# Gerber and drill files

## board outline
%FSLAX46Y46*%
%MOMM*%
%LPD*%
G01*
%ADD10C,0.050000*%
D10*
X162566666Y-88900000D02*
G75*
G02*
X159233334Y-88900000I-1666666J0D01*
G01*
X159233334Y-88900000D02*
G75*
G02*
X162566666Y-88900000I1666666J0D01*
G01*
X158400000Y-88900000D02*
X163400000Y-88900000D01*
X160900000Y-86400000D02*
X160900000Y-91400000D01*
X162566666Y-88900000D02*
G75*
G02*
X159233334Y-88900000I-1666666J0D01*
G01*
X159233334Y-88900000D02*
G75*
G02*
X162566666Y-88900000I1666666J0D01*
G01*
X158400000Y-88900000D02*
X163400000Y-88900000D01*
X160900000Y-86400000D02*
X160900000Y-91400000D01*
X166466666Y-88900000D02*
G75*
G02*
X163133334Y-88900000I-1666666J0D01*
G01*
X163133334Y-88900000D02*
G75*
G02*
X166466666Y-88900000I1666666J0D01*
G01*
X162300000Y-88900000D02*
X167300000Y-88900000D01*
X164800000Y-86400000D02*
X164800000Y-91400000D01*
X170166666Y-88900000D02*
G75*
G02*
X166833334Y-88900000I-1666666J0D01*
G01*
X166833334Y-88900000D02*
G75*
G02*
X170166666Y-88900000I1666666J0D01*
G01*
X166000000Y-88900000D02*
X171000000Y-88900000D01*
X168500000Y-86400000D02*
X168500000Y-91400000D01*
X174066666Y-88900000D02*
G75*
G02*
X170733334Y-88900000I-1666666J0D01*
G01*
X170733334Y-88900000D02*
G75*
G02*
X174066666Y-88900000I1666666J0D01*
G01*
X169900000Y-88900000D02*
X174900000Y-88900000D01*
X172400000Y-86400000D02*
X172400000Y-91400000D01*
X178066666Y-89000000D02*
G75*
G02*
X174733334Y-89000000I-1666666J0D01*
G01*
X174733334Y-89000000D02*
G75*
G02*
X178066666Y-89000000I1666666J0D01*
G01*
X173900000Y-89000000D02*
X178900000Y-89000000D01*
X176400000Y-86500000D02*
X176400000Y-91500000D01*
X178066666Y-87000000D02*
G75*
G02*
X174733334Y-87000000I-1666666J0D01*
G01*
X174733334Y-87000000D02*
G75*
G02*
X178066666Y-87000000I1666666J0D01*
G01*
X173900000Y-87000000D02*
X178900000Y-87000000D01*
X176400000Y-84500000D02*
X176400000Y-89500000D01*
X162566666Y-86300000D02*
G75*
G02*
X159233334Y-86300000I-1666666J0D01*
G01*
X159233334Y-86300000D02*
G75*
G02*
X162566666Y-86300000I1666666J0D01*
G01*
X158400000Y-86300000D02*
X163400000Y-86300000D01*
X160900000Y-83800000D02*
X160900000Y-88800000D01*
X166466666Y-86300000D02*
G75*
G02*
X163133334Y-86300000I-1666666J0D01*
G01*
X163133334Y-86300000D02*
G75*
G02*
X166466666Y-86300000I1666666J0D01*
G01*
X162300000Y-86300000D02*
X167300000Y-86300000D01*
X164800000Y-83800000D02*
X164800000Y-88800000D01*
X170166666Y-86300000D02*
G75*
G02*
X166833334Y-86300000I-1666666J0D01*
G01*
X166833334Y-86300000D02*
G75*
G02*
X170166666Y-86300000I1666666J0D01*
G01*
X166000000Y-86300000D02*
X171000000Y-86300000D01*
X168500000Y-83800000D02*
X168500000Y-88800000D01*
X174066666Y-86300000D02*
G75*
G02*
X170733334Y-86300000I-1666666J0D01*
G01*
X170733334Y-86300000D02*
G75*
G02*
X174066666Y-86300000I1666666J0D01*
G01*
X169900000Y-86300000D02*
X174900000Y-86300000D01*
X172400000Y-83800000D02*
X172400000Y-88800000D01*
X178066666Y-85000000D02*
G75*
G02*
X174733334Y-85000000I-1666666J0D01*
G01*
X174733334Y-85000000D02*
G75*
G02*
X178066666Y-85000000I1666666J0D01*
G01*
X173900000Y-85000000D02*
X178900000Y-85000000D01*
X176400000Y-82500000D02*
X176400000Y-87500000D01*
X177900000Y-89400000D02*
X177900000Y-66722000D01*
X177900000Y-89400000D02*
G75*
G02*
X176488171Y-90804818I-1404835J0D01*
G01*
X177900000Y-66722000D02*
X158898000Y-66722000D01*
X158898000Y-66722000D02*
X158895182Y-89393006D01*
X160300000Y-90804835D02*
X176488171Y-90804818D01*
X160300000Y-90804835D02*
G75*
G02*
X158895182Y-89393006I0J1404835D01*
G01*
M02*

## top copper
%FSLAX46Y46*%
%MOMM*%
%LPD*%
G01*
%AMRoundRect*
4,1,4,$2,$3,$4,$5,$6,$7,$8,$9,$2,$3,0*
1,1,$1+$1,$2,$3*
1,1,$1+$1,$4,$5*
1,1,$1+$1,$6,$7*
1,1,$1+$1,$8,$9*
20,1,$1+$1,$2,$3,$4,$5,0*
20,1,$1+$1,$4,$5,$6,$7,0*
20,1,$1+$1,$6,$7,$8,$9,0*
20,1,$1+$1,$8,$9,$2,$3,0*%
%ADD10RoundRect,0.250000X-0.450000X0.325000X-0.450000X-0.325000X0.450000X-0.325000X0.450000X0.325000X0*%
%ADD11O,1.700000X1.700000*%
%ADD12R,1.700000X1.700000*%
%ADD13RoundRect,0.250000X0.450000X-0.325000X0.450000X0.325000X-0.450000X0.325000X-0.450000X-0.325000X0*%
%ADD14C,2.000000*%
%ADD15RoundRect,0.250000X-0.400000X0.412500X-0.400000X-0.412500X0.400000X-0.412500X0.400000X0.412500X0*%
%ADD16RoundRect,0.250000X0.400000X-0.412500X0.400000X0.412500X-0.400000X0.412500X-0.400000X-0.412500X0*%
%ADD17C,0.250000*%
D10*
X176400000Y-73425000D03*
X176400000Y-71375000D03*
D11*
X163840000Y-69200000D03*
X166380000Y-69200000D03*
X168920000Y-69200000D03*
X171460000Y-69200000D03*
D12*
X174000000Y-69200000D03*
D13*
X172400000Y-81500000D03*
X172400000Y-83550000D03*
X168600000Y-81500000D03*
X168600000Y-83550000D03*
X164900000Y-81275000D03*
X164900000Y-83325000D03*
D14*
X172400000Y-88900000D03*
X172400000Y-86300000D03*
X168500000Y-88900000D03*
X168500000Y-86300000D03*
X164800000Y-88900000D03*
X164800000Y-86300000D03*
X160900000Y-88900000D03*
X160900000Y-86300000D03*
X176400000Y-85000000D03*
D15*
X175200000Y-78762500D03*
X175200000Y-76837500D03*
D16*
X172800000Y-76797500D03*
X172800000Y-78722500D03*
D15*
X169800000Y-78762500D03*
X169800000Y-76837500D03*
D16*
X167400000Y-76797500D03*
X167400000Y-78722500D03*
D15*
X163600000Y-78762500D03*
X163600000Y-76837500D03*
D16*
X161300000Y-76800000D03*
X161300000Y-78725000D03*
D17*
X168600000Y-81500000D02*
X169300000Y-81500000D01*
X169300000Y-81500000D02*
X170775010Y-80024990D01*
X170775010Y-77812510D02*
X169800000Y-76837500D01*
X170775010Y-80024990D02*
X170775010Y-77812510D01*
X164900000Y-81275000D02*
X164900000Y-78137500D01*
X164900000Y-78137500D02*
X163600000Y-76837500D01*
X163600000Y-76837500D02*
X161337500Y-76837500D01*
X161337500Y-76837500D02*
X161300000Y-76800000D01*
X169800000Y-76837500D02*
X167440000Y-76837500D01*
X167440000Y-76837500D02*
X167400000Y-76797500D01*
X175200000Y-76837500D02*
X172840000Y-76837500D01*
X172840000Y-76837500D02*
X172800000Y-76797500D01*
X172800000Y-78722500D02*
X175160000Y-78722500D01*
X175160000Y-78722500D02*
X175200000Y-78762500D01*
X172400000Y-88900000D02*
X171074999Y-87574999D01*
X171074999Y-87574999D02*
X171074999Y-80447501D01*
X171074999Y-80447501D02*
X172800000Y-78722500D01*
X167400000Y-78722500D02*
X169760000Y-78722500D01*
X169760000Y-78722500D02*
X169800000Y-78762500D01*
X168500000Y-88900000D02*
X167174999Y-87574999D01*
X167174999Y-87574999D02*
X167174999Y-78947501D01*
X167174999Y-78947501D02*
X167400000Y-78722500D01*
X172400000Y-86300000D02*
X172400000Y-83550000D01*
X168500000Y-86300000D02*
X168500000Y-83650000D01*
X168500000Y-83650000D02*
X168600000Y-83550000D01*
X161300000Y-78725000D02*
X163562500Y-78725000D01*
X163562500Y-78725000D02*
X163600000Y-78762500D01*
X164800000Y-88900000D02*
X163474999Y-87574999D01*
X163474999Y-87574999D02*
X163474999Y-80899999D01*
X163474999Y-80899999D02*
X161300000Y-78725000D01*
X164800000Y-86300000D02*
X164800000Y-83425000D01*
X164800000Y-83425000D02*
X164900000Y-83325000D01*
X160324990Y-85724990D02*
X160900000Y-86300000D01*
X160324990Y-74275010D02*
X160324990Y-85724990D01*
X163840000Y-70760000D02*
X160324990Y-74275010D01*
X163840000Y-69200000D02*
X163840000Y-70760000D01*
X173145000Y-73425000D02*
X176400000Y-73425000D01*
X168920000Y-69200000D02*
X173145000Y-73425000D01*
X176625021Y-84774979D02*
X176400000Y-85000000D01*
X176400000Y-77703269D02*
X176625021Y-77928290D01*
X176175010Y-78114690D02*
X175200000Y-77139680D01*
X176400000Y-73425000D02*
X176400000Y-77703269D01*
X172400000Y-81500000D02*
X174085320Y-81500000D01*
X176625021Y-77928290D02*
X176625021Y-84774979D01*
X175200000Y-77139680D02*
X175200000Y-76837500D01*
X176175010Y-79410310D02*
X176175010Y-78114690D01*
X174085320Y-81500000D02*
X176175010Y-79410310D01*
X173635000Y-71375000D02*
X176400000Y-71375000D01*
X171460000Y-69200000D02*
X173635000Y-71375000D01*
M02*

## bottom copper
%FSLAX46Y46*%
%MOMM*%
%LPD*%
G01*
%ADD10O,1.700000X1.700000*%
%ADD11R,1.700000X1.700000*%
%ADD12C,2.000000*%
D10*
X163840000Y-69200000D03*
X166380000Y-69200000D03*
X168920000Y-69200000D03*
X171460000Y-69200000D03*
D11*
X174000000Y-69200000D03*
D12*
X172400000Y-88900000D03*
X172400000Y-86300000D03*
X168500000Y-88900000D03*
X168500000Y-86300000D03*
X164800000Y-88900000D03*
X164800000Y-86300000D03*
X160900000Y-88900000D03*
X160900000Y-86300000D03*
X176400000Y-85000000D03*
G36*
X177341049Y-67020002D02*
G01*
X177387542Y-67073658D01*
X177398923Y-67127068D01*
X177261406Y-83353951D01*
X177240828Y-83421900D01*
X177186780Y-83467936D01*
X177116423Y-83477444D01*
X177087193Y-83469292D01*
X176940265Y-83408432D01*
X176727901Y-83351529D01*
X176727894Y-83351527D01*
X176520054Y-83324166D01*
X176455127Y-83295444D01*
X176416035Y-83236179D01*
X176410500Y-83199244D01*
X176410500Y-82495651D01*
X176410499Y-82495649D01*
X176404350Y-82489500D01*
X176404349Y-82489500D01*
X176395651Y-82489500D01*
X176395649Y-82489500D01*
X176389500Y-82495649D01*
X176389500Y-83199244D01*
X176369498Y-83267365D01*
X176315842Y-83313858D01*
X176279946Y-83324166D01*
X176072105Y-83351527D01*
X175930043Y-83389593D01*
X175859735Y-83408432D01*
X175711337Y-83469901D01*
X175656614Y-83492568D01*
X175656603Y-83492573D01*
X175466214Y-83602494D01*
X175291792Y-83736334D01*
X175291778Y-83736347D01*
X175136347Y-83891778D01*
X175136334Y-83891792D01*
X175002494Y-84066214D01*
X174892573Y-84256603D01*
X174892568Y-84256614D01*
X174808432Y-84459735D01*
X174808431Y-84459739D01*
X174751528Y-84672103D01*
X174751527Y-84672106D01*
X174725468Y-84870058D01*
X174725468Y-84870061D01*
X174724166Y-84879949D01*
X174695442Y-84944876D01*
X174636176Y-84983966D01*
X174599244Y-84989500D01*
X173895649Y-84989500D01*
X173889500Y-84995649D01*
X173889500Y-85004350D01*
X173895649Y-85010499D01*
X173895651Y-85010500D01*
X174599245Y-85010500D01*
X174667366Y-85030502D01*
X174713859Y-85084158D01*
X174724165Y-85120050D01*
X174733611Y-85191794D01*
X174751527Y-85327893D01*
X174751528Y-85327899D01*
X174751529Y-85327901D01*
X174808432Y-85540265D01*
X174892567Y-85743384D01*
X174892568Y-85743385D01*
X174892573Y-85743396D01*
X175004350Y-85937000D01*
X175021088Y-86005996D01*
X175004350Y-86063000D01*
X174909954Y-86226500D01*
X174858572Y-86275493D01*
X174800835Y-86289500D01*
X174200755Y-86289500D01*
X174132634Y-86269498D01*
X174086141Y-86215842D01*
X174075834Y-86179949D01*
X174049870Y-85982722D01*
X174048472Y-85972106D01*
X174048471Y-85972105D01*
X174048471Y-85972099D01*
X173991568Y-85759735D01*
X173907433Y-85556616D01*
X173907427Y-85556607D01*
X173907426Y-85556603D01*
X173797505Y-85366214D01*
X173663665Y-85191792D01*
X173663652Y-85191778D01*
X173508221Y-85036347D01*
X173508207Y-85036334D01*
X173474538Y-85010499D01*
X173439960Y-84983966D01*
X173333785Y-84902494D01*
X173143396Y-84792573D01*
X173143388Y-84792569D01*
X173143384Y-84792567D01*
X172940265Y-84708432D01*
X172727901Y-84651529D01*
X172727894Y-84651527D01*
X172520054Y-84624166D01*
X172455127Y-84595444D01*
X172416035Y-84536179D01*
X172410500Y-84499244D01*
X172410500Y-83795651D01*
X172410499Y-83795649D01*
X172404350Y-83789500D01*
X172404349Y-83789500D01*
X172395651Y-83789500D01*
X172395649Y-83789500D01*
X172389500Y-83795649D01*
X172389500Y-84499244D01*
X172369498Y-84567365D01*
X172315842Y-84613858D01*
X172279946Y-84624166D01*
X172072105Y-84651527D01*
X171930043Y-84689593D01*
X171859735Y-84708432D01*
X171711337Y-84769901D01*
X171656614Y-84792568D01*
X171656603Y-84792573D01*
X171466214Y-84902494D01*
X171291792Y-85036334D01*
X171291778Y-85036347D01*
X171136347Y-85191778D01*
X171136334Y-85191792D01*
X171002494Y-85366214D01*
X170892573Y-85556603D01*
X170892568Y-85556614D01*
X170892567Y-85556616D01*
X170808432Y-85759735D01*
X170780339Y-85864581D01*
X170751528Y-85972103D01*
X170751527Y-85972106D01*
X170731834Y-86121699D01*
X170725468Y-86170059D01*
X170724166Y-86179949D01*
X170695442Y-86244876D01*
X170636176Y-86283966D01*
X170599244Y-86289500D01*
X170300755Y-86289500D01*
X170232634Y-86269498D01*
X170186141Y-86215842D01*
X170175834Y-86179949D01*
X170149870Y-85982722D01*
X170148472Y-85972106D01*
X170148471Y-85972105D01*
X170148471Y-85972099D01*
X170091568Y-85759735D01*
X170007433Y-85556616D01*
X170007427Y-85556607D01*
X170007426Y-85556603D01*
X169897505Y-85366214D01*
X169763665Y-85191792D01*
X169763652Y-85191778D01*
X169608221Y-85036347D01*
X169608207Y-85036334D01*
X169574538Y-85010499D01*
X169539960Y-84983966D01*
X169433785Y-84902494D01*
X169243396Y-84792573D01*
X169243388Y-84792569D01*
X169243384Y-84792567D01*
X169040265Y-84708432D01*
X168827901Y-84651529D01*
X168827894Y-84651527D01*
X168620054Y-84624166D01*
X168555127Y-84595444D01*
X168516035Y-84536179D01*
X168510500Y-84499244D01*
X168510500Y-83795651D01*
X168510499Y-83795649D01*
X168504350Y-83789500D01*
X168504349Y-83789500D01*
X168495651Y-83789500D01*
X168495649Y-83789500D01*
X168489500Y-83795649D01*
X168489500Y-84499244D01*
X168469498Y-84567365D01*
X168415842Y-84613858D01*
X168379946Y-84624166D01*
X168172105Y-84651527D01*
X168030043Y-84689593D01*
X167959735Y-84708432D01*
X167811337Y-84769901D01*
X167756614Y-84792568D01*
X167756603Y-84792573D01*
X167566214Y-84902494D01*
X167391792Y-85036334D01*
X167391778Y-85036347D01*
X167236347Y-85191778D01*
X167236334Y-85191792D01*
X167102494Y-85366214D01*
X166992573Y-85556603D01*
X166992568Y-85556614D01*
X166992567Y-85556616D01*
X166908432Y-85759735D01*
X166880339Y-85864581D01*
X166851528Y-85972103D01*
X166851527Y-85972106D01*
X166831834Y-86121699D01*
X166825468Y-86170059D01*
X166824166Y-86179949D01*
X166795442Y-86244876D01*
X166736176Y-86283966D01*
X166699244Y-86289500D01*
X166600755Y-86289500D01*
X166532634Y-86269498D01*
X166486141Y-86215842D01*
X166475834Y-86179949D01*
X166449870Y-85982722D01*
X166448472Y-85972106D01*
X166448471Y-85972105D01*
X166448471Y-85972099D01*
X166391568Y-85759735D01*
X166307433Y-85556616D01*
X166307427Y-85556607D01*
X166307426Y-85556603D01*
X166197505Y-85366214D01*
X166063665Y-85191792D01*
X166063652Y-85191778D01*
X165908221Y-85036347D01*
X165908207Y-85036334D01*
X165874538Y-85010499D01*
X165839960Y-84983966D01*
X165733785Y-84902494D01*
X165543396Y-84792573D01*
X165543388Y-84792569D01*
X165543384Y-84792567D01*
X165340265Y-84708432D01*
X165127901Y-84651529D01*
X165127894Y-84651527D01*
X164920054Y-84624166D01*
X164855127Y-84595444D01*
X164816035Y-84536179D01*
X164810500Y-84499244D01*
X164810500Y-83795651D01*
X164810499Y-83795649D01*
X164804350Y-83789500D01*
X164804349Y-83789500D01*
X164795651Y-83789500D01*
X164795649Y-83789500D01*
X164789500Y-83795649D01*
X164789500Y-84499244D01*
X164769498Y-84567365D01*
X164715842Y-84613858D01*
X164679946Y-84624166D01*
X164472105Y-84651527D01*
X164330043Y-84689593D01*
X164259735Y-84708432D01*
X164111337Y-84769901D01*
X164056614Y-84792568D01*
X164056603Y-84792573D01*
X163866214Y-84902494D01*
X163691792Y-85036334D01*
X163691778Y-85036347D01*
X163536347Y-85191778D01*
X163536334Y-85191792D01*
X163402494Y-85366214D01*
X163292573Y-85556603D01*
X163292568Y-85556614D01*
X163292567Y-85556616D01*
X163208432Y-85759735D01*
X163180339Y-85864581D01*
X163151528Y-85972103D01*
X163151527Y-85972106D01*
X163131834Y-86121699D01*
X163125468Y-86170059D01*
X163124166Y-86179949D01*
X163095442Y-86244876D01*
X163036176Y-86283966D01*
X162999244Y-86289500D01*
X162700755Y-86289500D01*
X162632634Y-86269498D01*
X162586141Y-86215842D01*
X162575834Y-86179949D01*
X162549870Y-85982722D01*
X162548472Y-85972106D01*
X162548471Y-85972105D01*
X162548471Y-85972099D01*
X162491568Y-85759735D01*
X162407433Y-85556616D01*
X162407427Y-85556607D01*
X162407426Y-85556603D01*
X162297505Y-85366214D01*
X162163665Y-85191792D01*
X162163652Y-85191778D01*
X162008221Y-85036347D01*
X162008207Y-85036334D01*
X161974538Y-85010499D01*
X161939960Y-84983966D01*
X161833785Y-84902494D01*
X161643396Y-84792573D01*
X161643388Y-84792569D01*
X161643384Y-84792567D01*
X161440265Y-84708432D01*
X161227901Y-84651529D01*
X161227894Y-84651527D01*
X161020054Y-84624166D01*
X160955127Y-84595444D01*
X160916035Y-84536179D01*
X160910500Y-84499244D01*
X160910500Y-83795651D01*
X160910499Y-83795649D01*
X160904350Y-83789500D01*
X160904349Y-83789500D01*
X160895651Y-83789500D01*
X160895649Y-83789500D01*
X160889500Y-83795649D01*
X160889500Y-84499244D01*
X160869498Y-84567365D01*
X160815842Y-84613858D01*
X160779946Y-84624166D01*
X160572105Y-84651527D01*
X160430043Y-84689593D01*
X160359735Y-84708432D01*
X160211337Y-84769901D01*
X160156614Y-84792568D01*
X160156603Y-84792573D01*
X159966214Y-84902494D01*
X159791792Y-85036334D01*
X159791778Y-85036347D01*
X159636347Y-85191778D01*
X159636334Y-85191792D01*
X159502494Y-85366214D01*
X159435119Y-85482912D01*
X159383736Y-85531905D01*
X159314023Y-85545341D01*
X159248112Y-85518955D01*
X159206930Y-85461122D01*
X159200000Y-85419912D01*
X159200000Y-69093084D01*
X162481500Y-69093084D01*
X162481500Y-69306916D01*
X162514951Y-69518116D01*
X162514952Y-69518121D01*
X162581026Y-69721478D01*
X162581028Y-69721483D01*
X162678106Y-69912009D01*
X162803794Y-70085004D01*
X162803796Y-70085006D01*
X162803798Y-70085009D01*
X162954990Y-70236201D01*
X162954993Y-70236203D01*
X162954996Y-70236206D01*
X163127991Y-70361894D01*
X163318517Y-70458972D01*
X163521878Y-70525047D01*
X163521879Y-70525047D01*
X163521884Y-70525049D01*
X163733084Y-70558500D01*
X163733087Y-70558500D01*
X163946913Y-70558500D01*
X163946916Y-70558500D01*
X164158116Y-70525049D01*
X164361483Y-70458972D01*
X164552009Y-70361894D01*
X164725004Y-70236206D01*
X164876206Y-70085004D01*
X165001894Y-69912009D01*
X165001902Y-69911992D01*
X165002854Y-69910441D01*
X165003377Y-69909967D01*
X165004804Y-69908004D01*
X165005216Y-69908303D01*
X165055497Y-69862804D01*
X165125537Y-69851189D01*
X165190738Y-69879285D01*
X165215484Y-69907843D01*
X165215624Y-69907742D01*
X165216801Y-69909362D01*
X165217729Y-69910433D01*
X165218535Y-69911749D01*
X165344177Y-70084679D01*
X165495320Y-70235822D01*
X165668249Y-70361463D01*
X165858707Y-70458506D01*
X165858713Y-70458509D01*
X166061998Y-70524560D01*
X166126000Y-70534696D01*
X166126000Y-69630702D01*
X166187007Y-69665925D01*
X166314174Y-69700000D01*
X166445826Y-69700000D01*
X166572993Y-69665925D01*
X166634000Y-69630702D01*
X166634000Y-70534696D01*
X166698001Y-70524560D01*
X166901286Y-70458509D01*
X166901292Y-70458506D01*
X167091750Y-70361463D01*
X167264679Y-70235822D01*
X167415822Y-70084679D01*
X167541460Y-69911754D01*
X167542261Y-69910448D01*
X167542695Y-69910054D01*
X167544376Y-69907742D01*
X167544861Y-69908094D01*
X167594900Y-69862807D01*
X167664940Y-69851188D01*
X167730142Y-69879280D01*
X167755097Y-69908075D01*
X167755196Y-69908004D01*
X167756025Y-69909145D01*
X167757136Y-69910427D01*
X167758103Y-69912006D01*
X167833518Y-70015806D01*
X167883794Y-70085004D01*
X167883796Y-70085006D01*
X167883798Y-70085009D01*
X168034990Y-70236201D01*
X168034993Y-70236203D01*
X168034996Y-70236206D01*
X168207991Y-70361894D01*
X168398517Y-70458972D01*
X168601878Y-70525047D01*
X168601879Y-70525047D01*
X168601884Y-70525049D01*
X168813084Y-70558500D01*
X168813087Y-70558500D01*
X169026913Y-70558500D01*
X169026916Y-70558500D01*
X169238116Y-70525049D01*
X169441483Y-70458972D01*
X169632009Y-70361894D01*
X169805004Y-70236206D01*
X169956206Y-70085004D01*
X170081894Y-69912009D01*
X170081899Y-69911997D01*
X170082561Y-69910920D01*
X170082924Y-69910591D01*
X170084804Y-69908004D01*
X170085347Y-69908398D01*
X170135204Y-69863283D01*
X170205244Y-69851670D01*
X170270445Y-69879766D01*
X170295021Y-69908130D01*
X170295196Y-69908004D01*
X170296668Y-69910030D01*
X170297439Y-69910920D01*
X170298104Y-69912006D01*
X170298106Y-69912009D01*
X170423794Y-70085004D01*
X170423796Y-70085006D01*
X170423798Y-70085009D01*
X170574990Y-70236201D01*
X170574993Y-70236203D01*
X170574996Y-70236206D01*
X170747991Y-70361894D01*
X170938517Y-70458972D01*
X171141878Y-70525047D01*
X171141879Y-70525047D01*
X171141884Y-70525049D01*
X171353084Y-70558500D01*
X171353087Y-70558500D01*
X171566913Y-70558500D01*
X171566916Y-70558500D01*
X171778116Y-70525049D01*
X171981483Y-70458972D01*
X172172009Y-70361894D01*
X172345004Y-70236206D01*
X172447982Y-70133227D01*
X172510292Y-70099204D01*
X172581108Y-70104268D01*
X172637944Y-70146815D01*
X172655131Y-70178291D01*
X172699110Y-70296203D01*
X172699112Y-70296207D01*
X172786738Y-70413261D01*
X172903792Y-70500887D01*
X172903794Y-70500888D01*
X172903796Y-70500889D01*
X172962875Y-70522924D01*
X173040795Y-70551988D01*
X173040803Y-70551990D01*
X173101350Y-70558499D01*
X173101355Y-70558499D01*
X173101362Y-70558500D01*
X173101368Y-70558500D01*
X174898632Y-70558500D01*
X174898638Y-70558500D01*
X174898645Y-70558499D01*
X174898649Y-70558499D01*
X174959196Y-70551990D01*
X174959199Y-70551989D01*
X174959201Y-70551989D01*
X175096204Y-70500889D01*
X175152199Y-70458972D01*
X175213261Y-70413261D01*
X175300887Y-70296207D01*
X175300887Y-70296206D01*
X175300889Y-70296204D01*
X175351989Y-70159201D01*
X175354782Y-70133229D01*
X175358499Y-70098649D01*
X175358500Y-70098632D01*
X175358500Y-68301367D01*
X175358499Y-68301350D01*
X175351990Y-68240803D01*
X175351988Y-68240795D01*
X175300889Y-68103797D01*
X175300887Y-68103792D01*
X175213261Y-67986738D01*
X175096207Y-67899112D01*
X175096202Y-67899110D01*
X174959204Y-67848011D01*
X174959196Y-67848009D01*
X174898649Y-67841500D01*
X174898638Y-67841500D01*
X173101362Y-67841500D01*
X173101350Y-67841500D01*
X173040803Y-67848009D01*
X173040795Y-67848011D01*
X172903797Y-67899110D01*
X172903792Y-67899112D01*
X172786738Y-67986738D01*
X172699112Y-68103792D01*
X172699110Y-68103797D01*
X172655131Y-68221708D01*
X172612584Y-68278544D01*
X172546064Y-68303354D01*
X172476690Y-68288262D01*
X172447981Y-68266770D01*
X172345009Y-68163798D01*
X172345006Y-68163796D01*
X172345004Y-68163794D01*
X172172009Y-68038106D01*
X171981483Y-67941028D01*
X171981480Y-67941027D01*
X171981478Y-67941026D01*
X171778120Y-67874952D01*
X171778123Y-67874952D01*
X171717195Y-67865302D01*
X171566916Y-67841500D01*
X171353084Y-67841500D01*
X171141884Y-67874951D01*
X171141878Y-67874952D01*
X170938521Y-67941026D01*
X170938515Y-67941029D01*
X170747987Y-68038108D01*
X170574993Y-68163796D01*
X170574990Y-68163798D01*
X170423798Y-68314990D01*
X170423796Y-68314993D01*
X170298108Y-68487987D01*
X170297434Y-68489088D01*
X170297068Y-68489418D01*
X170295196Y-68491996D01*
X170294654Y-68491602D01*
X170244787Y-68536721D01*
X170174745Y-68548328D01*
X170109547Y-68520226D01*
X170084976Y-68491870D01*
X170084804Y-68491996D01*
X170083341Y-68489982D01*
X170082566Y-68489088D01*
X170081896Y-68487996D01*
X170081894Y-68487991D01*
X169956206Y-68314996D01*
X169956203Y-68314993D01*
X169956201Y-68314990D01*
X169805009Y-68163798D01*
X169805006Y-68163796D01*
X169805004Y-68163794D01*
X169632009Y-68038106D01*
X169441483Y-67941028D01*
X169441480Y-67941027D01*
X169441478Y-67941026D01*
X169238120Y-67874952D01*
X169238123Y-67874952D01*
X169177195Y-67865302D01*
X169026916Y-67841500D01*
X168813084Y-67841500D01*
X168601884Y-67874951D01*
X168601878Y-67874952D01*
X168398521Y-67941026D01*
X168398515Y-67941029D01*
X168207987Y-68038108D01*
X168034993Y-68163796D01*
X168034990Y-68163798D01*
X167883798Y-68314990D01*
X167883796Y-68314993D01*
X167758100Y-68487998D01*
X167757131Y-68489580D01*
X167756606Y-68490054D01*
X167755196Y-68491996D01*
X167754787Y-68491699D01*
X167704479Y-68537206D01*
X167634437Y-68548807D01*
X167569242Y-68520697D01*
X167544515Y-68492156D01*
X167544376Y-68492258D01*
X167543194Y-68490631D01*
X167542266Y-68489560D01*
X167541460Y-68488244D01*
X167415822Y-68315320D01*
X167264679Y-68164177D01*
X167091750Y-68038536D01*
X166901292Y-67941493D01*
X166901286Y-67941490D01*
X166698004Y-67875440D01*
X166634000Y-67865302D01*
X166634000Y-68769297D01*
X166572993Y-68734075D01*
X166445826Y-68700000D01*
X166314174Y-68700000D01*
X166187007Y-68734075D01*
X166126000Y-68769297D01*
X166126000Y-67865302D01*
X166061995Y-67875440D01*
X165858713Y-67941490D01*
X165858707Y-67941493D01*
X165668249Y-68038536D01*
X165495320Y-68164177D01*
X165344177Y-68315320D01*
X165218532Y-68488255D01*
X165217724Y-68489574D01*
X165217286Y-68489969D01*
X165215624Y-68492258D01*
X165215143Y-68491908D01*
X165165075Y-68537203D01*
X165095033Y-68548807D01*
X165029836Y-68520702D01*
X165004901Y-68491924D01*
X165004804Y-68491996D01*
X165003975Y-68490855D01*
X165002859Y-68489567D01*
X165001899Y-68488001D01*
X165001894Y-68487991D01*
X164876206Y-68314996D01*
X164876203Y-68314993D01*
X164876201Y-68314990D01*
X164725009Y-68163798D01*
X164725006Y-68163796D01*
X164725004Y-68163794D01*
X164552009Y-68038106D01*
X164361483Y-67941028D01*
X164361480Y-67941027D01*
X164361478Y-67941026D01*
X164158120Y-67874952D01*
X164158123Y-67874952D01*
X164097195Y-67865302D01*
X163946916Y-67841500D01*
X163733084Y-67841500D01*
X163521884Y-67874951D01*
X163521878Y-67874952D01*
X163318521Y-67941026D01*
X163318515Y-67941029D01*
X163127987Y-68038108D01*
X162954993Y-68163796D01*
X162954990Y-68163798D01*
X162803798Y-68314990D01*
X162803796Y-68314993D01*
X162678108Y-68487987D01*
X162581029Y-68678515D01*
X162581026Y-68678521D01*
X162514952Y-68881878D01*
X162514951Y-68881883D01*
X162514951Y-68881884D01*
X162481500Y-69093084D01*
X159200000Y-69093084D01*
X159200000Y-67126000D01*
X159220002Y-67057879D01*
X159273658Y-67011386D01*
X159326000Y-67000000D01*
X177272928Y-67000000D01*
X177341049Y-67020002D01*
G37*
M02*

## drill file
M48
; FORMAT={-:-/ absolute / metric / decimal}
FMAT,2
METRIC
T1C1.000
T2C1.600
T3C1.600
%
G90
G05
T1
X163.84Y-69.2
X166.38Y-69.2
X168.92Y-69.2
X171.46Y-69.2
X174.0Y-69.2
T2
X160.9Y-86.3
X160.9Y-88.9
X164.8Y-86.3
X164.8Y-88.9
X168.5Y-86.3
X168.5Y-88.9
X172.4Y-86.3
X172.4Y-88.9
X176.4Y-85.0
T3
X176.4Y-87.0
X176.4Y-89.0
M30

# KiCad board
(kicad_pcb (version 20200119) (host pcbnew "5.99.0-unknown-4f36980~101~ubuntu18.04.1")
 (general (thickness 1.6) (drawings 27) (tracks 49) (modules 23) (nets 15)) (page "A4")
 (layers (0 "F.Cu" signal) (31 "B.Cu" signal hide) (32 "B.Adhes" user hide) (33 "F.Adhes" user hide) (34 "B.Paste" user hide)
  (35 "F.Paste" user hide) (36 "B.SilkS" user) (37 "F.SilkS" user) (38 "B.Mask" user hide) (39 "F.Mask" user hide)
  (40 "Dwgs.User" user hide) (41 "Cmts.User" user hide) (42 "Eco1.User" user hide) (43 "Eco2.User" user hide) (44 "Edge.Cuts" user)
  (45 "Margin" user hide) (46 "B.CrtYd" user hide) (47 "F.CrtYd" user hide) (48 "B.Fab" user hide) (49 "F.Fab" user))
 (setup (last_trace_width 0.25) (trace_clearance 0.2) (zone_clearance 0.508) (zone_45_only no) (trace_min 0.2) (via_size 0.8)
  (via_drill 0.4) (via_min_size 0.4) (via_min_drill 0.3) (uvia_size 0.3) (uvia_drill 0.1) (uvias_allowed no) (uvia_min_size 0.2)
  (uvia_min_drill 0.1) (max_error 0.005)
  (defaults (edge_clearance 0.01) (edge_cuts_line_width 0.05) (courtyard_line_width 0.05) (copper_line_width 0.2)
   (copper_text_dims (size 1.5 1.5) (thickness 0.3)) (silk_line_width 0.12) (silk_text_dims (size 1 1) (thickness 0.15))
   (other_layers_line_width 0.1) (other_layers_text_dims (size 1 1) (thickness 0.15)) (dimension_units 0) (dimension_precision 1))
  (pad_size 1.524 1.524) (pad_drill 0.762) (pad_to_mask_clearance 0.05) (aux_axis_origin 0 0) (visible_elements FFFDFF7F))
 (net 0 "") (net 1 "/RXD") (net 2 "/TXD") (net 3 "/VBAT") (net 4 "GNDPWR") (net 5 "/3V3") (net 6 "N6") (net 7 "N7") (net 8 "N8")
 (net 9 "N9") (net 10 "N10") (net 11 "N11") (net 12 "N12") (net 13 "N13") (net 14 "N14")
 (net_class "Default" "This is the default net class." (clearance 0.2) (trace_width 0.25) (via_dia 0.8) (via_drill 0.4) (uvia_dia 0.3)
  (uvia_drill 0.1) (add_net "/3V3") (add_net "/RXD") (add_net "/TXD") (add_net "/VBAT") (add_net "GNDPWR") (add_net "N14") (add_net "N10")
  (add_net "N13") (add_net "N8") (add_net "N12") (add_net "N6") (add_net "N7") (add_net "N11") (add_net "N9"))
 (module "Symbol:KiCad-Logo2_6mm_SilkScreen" (layer "B.Cu") (at 168.4 79.4 180)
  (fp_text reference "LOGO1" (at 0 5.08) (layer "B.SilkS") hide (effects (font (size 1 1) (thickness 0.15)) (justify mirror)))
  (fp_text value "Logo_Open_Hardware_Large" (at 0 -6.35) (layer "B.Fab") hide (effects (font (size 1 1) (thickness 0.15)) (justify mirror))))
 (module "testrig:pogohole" (layer "F.Cu") (at 176.4 89)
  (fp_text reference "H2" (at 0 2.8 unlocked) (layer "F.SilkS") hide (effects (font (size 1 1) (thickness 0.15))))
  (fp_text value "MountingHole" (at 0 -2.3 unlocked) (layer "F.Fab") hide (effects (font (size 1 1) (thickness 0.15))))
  (pad "" np_thru_hole circle (at 0 0) (size 1.6 1.6) (drill 1.6) (layers *.Cu *.Mask) (solder_mask_margin 0.3) (clearance 0.3)))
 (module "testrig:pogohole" (layer "F.Cu") (at 176.4 87)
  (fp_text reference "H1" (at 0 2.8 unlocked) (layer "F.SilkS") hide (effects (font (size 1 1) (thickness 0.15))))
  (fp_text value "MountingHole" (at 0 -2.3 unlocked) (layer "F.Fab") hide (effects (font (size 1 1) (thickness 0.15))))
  (pad "" np_thru_hole circle (at 0 0) (size 1.6 1.6) (drill 1.6) (layers *.Cu *.Mask) (solder_mask_margin 0.3) (clearance 0.3)))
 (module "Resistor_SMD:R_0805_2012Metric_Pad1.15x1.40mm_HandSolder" (layer "F.Cu") (at 176.4 72.4 -90)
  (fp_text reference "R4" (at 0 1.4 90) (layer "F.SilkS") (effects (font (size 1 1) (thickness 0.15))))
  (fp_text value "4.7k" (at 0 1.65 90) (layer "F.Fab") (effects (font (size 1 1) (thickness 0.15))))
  (pad "2" smd roundrect (at 1.025 0 270) (size 1.15 1.4) (layers "F.Cu" "F.Paste" "F.Mask") (roundrect_rratio 0.217391) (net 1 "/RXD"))
  (pad "1" smd roundrect (at -1.025 0 270) (size 1.15 1.4) (layers "F.Cu" "F.Paste" "F.Mask") (roundrect_rratio 0.217391) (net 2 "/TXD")))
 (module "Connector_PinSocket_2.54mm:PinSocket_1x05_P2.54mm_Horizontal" (layer "F.Cu") (at 174 69.2 -90)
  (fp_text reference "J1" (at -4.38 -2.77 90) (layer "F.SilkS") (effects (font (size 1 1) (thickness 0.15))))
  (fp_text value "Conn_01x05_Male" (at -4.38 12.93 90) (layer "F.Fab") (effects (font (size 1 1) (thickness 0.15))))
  (pad "5" thru_hole oval (at 0 10.16 270) (size 1.7 1.7) (drill 1) (layers *.Cu *.Mask) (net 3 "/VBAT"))
  (pad "4" thru_hole oval (at 0 7.62 270) (size 1.7 1.7) (drill 1) (layers *.Cu *.Mask) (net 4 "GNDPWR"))
  (pad "3" thru_hole oval (at 0 5.08 270) (size 1.7 1.7) (drill 1) (layers *.Cu *.Mask) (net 1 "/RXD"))
  (pad "2" thru_hole oval (at 0 2.54 270) (size 1.7 1.7) (drill 1) (layers *.Cu *.Mask) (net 2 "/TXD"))
  (pad "1" thru_hole rect (at 0 0 270) (size 1.7 1.7) (drill 1) (layers *.Cu *.Mask) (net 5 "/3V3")))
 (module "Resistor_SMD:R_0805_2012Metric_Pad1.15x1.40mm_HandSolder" (layer "F.Cu") (at 172.4 82.525 90)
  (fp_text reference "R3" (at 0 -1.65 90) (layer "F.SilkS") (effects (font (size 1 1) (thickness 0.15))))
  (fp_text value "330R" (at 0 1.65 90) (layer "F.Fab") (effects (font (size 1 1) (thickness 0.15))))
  (pad "2" smd roundrect (at 1.025 0 90) (size 1.15 1.4) (layers "F.Cu" "F.Paste" "F.Mask") (roundrect_rratio 0.217391) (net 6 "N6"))
  (pad "1" smd roundrect (at -1.025 0 90) (size 1.15 1.4) (layers "F.Cu" "F.Paste" "F.Mask") (roundrect_rratio 0.217391) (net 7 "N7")))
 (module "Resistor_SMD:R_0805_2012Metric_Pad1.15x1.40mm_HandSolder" (layer "F.Cu") (at 168.6 82.525 90)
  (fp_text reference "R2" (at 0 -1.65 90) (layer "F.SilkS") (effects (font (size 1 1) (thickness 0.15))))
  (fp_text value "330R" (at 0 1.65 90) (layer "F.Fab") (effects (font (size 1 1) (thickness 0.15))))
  (pad "2" smd roundrect (at 1.025 0 90) (size 1.15 1.4) (layers "F.Cu" "F.Paste" "F.Mask") (roundrect_rratio 0.217391) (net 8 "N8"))
  (pad "1" smd roundrect (at -1.025 0 90) (size 1.15 1.4) (layers "F.Cu" "F.Paste" "F.Mask") (roundrect_rratio 0.217391) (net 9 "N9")))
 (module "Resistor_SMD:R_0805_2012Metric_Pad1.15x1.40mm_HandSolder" (layer "F.Cu") (at 164.9 82.3 90)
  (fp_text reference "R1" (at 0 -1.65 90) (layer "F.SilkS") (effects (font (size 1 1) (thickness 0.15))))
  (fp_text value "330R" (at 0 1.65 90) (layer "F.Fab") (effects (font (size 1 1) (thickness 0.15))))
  (pad "2" smd roundrect (at 1.025 0 90) (size 1.15 1.4) (layers "F.Cu" "F.Paste" "F.Mask") (roundrect_rratio 0.217391) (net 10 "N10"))
  (pad "1" smd roundrect (at -1.025 0 90) (size 1.15 1.4) (layers "F.Cu" "F.Paste" "F.Mask") (roundrect_rratio 0.217391) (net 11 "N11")))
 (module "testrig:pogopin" (layer "F.Cu") (at 172.4 88.9)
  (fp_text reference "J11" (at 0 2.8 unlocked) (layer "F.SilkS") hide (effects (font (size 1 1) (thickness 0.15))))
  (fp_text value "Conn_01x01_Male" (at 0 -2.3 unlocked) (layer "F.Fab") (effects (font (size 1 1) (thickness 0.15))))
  (pad "1" thru_hole circle (at 0 0) (size 2 2) (drill 1.6) (layers *.Cu *.Mask) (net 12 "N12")))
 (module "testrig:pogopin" (layer "F.Cu") (at 172.4 86.3)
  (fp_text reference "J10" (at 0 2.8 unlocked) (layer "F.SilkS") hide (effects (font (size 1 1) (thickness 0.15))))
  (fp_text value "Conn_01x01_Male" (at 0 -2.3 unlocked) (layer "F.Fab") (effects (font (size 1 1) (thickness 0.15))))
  (pad "1" thru_hole circle (at 0 0) (size 2 2) (drill 1.6) (layers *.Cu *.Mask) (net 7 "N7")))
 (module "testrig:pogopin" (layer "F.Cu") (at 168.5 88.9)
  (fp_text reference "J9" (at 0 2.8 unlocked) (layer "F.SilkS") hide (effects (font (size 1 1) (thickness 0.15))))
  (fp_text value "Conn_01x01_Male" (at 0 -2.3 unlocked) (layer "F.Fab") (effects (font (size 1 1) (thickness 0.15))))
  (pad "1" thru_hole circle (at 0 0) (size 2 2) (drill 1.6) (layers *.Cu *.Mask) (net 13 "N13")))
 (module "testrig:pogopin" (layer "F.Cu") (at 168.5 86.3)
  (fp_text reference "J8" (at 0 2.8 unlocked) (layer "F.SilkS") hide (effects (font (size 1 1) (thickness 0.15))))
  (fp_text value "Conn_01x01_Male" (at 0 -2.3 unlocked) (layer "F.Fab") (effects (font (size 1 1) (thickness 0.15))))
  (pad "1" thru_hole circle (at 0 0) (size 2 2) (drill 1.6) (layers *.Cu *.Mask) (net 9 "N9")))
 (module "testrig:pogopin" (layer "F.Cu") (at 164.8 88.9)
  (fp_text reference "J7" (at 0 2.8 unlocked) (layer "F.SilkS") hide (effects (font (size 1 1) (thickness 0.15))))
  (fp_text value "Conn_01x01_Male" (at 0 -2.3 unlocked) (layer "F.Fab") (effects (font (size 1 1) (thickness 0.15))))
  (pad "1" thru_hole circle (at 0 0) (size 2 2) (drill 1.6) (layers *.Cu *.Mask) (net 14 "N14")))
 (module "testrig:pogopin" (layer "F.Cu") (at 164.8 86.3)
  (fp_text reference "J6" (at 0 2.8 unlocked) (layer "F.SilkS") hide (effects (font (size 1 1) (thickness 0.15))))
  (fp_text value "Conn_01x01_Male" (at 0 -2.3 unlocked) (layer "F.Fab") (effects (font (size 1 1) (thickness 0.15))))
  (pad "1" thru_hole circle (at 0 0) (size 2 2) (drill 1.6) (layers *.Cu *.Mask) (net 11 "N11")))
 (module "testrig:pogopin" (layer "F.Cu") (at 160.9 88.9)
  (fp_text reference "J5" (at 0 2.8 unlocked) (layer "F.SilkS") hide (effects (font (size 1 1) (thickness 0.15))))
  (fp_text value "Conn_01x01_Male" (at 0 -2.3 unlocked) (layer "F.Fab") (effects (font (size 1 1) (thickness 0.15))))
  (pad "1" thru_hole circle (at 0 0) (size 2 2) (drill 1.6) (layers *.Cu *.Mask) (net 4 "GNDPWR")))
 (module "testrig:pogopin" (layer "F.Cu") (at 160.9 86.3)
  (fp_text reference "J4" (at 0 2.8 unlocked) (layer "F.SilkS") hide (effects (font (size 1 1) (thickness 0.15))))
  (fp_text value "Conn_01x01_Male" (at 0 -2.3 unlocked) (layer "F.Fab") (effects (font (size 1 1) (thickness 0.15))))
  (pad "1" thru_hole circle (at 0 0) (size 2 2) (drill 1.6) (layers *.Cu *.Mask) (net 3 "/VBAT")))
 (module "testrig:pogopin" (layer "F.Cu") (at 176.4 85)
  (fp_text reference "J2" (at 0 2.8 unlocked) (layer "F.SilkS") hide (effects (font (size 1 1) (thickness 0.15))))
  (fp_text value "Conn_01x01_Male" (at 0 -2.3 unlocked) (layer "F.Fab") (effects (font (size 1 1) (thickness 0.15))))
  (pad "1" thru_hole circle (at 0 0) (size 2 2) (drill 1.6) (layers *.Cu *.Mask) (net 1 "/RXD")))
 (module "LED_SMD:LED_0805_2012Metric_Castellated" (layer "F.Cu") (at 175.2 77.8 -90)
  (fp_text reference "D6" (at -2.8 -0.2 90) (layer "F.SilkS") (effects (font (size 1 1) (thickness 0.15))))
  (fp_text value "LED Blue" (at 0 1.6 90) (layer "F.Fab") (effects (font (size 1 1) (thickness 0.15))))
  (pad "2" smd roundrect (at 0.9625 0 270) (size 1.325 1.3) (layers "F.Cu" "F.Paste" "F.Mask") (roundrect_rratio 0.192308) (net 12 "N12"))
  (pad "1" smd roundrect (at -0.9625 0 270) (size 1.325 1.3) (layers "F.Cu" "F.Paste" "F.Mask") (roundrect_rratio 0.192308) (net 6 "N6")))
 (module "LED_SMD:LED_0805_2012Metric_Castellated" (layer "F.Cu") (at 172.8 77.76 90)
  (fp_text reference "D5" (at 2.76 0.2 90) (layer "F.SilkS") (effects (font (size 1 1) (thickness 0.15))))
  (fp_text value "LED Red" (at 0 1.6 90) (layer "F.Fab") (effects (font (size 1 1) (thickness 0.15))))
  (pad "2" smd roundrect (at 0.9625 0 90) (size 1.325 1.3) (layers "F.Cu" "F.Paste" "F.Mask") (roundrect_rratio 0.192308) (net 6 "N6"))
  (pad "1" smd roundrect (at -0.9625 0 90) (size 1.325 1.3) (layers "F.Cu" "F.Paste" "F.Mask") (roundrect_rratio 0.192308) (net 12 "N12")))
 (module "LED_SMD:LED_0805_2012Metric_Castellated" (layer "F.Cu") (at 169.8 77.8 -90)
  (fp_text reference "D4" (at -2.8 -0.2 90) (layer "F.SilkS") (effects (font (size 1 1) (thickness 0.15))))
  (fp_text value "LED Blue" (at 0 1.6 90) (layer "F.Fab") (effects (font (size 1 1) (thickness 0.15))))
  (pad "2" smd roundrect (at 0.9625 0 270) (size 1.325 1.3) (layers "F.Cu" "F.Paste" "F.Mask") (roundrect_rratio 0.192308) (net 13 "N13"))
  (pad "1" smd roundrect (at -0.9625 0 270) (size 1.325 1.3) (layers "F.Cu" "F.Paste" "F.Mask") (roundrect_rratio 0.192308) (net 8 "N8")))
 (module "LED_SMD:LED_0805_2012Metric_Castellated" (layer "F.Cu") (at 167.4 77.76 90)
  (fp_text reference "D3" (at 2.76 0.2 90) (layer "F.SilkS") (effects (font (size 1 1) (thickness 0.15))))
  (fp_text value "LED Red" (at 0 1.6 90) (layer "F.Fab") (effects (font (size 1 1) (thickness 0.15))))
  (pad "2" smd roundrect (at 0.9625 0 90) (size 1.325 1.3) (layers "F.Cu" "F.Paste" "F.Mask") (roundrect_rratio 0.192308) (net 8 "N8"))
  (pad "1" smd roundrect (at -0.9625 0 90) (size 1.325 1.3) (layers "F.Cu" "F.Paste" "F.Mask") (roundrect_rratio 0.192308) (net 13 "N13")))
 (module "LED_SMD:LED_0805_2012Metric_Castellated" (layer "F.Cu") (at 163.6 77.8 -90)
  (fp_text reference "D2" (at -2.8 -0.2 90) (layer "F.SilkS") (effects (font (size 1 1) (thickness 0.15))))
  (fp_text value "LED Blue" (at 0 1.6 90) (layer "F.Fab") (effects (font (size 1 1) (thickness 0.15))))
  (pad "2" smd roundrect (at 0.9625 0 270) (size 1.325 1.3) (layers "F.Cu" "F.Paste" "F.Mask") (roundrect_rratio 0.192308) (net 14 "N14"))
  (pad "1" smd roundrect (at -0.9625 0 270) (size 1.325 1.3) (layers "F.Cu" "F.Paste" "F.Mask") (roundrect_rratio 0.192308) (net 10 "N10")))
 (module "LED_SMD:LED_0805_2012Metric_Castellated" (layer "F.Cu") (at 161.3 77.7625 90)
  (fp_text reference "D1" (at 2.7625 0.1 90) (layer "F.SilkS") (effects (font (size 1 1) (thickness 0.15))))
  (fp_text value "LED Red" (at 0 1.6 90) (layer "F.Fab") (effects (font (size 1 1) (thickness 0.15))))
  (pad "2" smd roundrect (at 0.9625 0 90) (size 1.325 1.3) (layers "F.Cu" "F.Paste" "F.Mask") (roundrect_rratio 0.192308) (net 10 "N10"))
  (pad "1" smd roundrect (at -0.9625 0 90) (size 1.325 1.3) (layers "F.Cu" "F.Paste" "F.Mask") (roundrect_rratio 0.192308) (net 14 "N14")))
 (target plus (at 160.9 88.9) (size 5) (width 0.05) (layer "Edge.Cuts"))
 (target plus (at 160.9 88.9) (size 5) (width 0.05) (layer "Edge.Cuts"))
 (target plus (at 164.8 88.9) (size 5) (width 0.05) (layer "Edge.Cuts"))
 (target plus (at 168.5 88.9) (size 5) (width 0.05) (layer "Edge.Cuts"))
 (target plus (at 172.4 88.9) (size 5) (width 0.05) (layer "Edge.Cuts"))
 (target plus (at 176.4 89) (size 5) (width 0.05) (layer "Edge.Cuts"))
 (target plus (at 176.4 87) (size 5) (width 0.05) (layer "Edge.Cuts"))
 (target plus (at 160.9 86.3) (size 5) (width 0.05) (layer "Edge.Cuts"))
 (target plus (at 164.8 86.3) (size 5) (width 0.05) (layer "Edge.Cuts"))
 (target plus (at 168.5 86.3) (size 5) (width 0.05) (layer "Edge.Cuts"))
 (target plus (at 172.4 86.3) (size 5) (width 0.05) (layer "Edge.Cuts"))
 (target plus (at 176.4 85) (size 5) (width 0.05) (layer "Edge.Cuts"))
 (gr_line (start 177.9 89.4) (end 177.9 66.722) (layer "Edge.Cuts") (width 0.05))
 (gr_arc (start 176.495165 89.4) (end 176.488171 90.804818) (angle -90.28524931) (layer "Edge.Cuts") (width 0.05))
 (gr_line (start 177.9 66.722) (end 158.898 66.722) (layer "Edge.Cuts") (width 0.05))
 (gr_line (start 158.898 66.722) (end 158.895182 89.393006) (layer "Edge.Cuts") (width 0.05))
 (gr_line (start 160.3 90.804835) (end 176.488171 90.804818) (layer "Edge.Cuts") (width 0.05))
 (gr_arc (start 160.3 89.4) (end 158.895182 89.393006) (angle -90.28524931) (layer "Edge.Cuts") (width 0.05))
 (segment (start 168.6 81.5) (end 169.3 81.5) (width 0.25) (layer "F.Cu") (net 8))
 (segment (start 169.3 81.5) (end 170.77501 80.02499) (width 0.25) (layer "F.Cu") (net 8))
 (segment (start 170.77501 77.81251) (end 169.8 76.8375) (width 0.25) (layer "F.Cu") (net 8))
 (segment (start 170.77501 80.02499) (end 170.77501 77.81251) (width 0.25) (layer "F.Cu") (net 8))
 (segment (start 164.9 81.275) (end 164.9 78.1375) (width 0.25) (layer "F.Cu") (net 10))
 (segment (start 164.9 78.1375) (end 163.6 76.8375) (width 0.25) (layer "F.Cu") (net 10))
 (segment (start 163.6 76.8375) (end 161.3375 76.8375) (width 0.25) (layer "F.Cu") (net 10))
 (segment (start 161.3375 76.8375) (end 161.3 76.8) (width 0.25) (layer "F.Cu") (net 10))
 (segment (start 169.8 76.8375) (end 167.44 76.8375) (width 0.25) (layer "F.Cu") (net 8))
 (segment (start 167.44 76.8375) (end 167.4 76.7975) (width 0.25) (layer "F.Cu") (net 8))
 (segment (start 175.2 76.8375) (end 172.84 76.8375) (width 0.25) (layer "F.Cu") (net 6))
 (segment (start 172.84 76.8375) (end 172.8 76.7975) (width 0.25) (layer "F.Cu") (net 6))
 (segment (start 172.8 78.7225) (end 175.16 78.7225) (width 0.25) (layer "F.Cu") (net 12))
 (segment (start 175.16 78.7225) (end 175.2 78.7625) (width 0.25) (layer "F.Cu") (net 12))
 (segment (start 172.4 88.9) (end 171.074999 87.574999) (width 0.25) (layer "F.Cu") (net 12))
 (segment (start 171.074999 87.574999) (end 171.074999 80.447501) (width 0.25) (layer "F.Cu") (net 12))
 (segment (start 171.074999 80.447501) (end 172.8 78.7225) (width 0.25) (layer "F.Cu") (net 12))
 (segment (start 167.4 78.7225) (end 169.76 78.7225) (width 0.25) (layer "F.Cu") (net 13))
 (segment (start 169.76 78.7225) (end 169.8 78.7625) (width 0.25) (layer "F.Cu") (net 13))
 (segment (start 168.5 88.9) (end 167.174999 87.574999) (width 0.25) (layer "F.Cu") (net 13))
 (segment (start 167.174999 87.574999) (end 167.174999 78.947501) (width 0.25) (layer "F.Cu") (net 13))
 (segment (start 167.174999 78.947501) (end 167.4 78.7225) (width 0.25) (layer "F.Cu") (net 13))
 (segment (start 172.4 86.3) (end 172.4 83.55) (width 0.25) (layer "F.Cu") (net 7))
 (segment (start 168.5 86.3) (end 168.5 83.65) (width 0.25) (layer "F.Cu") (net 9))
 (segment (start 168.5 83.65) (end 168.6 83.55) (width 0.25) (layer "F.Cu") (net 9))
 (segment (start 161.3 78.725) (end 163.5625 78.725) (width 0.25) (layer "F.Cu") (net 14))
 (segment (start 163.5625 78.725) (end 163.6 78.7625) (width 0.25) (layer "F.Cu") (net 14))
 (segment (start 164.8 88.9) (end 163.474999 87.574999) (width 0.25) (layer "F.Cu") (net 14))
 (segment (start 163.474999 87.574999) (end 163.474999 80.899999) (width 0.25) (layer "F.Cu") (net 14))
 (segment (start 163.474999 80.899999) (end 161.3 78.725) (width 0.25) (layer "F.Cu") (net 14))
 (segment (start 164.8 86.3) (end 164.8 83.425) (width 0.25) (layer "F.Cu") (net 11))
 (segment (start 164.8 83.425) (end 164.9 83.325) (width 0.25) (layer "F.Cu") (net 11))
 (segment (start 160.32499 85.72499) (end 160.9 86.3) (width 0.25) (layer "F.Cu") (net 3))
 (segment (start 160.32499 74.27501) (end 160.32499 85.72499) (width 0.25) (layer "F.Cu") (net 3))
 (segment (start 163.84 70.76) (end 160.32499 74.27501) (width 0.25) (layer "F.Cu") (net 3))
 (segment (start 163.84 69.2) (end 163.84 70.76) (width 0.25) (layer "F.Cu") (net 3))
 (segment (start 173.145 73.425) (end 176.4 73.425) (width 0.25) (layer "F.Cu") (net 1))
 (segment (start 168.92 69.2) (end 173.145 73.425) (width 0.25) (layer "F.Cu") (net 1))
 (segment (start 176.625021 84.774979) (end 176.4 85) (width 0.25) (layer "F.Cu") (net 1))
 (segment (start 176.4 77.703269) (end 176.625021 77.92829) (width 0.25) (layer "F.Cu") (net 1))
 (segment (start 176.17501 78.11469) (end 175.2 77.13968) (width 0.25) (layer "F.Cu") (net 6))
 (segment (start 176.4 73.425) (end 176.4 77.703269) (width 0.25) (layer "F.Cu") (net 1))
 (segment (start 172.4 81.5) (end 174.08532 81.5) (width 0.25) (layer "F.Cu") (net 6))
 (segment (start 176.625021 77.92829) (end 176.625021 84.774979) (width 0.25) (layer "F.Cu") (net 1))
 (segment (start 175.2 77.13968) (end 175.2 76.8375) (width 0.25) (layer "F.Cu") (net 6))
 (segment (start 176.17501 79.41031) (end 176.17501 78.11469) (width 0.25) (layer "F.Cu") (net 6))
 (segment (start 174.08532 81.5) (end 176.17501 79.41031) (width 0.25) (layer "F.Cu") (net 6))
 (segment (start 173.635 71.375) (end 176.4 71.375) (width 0.25) (layer "F.Cu") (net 2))
 (segment (start 171.46 69.2) (end 173.635 71.375) (width 0.25) (layer "F.Cu") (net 2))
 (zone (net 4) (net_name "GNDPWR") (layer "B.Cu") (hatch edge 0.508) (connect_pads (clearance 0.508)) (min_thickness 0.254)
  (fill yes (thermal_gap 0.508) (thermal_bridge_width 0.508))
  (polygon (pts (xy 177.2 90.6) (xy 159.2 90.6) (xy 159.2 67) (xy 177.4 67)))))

